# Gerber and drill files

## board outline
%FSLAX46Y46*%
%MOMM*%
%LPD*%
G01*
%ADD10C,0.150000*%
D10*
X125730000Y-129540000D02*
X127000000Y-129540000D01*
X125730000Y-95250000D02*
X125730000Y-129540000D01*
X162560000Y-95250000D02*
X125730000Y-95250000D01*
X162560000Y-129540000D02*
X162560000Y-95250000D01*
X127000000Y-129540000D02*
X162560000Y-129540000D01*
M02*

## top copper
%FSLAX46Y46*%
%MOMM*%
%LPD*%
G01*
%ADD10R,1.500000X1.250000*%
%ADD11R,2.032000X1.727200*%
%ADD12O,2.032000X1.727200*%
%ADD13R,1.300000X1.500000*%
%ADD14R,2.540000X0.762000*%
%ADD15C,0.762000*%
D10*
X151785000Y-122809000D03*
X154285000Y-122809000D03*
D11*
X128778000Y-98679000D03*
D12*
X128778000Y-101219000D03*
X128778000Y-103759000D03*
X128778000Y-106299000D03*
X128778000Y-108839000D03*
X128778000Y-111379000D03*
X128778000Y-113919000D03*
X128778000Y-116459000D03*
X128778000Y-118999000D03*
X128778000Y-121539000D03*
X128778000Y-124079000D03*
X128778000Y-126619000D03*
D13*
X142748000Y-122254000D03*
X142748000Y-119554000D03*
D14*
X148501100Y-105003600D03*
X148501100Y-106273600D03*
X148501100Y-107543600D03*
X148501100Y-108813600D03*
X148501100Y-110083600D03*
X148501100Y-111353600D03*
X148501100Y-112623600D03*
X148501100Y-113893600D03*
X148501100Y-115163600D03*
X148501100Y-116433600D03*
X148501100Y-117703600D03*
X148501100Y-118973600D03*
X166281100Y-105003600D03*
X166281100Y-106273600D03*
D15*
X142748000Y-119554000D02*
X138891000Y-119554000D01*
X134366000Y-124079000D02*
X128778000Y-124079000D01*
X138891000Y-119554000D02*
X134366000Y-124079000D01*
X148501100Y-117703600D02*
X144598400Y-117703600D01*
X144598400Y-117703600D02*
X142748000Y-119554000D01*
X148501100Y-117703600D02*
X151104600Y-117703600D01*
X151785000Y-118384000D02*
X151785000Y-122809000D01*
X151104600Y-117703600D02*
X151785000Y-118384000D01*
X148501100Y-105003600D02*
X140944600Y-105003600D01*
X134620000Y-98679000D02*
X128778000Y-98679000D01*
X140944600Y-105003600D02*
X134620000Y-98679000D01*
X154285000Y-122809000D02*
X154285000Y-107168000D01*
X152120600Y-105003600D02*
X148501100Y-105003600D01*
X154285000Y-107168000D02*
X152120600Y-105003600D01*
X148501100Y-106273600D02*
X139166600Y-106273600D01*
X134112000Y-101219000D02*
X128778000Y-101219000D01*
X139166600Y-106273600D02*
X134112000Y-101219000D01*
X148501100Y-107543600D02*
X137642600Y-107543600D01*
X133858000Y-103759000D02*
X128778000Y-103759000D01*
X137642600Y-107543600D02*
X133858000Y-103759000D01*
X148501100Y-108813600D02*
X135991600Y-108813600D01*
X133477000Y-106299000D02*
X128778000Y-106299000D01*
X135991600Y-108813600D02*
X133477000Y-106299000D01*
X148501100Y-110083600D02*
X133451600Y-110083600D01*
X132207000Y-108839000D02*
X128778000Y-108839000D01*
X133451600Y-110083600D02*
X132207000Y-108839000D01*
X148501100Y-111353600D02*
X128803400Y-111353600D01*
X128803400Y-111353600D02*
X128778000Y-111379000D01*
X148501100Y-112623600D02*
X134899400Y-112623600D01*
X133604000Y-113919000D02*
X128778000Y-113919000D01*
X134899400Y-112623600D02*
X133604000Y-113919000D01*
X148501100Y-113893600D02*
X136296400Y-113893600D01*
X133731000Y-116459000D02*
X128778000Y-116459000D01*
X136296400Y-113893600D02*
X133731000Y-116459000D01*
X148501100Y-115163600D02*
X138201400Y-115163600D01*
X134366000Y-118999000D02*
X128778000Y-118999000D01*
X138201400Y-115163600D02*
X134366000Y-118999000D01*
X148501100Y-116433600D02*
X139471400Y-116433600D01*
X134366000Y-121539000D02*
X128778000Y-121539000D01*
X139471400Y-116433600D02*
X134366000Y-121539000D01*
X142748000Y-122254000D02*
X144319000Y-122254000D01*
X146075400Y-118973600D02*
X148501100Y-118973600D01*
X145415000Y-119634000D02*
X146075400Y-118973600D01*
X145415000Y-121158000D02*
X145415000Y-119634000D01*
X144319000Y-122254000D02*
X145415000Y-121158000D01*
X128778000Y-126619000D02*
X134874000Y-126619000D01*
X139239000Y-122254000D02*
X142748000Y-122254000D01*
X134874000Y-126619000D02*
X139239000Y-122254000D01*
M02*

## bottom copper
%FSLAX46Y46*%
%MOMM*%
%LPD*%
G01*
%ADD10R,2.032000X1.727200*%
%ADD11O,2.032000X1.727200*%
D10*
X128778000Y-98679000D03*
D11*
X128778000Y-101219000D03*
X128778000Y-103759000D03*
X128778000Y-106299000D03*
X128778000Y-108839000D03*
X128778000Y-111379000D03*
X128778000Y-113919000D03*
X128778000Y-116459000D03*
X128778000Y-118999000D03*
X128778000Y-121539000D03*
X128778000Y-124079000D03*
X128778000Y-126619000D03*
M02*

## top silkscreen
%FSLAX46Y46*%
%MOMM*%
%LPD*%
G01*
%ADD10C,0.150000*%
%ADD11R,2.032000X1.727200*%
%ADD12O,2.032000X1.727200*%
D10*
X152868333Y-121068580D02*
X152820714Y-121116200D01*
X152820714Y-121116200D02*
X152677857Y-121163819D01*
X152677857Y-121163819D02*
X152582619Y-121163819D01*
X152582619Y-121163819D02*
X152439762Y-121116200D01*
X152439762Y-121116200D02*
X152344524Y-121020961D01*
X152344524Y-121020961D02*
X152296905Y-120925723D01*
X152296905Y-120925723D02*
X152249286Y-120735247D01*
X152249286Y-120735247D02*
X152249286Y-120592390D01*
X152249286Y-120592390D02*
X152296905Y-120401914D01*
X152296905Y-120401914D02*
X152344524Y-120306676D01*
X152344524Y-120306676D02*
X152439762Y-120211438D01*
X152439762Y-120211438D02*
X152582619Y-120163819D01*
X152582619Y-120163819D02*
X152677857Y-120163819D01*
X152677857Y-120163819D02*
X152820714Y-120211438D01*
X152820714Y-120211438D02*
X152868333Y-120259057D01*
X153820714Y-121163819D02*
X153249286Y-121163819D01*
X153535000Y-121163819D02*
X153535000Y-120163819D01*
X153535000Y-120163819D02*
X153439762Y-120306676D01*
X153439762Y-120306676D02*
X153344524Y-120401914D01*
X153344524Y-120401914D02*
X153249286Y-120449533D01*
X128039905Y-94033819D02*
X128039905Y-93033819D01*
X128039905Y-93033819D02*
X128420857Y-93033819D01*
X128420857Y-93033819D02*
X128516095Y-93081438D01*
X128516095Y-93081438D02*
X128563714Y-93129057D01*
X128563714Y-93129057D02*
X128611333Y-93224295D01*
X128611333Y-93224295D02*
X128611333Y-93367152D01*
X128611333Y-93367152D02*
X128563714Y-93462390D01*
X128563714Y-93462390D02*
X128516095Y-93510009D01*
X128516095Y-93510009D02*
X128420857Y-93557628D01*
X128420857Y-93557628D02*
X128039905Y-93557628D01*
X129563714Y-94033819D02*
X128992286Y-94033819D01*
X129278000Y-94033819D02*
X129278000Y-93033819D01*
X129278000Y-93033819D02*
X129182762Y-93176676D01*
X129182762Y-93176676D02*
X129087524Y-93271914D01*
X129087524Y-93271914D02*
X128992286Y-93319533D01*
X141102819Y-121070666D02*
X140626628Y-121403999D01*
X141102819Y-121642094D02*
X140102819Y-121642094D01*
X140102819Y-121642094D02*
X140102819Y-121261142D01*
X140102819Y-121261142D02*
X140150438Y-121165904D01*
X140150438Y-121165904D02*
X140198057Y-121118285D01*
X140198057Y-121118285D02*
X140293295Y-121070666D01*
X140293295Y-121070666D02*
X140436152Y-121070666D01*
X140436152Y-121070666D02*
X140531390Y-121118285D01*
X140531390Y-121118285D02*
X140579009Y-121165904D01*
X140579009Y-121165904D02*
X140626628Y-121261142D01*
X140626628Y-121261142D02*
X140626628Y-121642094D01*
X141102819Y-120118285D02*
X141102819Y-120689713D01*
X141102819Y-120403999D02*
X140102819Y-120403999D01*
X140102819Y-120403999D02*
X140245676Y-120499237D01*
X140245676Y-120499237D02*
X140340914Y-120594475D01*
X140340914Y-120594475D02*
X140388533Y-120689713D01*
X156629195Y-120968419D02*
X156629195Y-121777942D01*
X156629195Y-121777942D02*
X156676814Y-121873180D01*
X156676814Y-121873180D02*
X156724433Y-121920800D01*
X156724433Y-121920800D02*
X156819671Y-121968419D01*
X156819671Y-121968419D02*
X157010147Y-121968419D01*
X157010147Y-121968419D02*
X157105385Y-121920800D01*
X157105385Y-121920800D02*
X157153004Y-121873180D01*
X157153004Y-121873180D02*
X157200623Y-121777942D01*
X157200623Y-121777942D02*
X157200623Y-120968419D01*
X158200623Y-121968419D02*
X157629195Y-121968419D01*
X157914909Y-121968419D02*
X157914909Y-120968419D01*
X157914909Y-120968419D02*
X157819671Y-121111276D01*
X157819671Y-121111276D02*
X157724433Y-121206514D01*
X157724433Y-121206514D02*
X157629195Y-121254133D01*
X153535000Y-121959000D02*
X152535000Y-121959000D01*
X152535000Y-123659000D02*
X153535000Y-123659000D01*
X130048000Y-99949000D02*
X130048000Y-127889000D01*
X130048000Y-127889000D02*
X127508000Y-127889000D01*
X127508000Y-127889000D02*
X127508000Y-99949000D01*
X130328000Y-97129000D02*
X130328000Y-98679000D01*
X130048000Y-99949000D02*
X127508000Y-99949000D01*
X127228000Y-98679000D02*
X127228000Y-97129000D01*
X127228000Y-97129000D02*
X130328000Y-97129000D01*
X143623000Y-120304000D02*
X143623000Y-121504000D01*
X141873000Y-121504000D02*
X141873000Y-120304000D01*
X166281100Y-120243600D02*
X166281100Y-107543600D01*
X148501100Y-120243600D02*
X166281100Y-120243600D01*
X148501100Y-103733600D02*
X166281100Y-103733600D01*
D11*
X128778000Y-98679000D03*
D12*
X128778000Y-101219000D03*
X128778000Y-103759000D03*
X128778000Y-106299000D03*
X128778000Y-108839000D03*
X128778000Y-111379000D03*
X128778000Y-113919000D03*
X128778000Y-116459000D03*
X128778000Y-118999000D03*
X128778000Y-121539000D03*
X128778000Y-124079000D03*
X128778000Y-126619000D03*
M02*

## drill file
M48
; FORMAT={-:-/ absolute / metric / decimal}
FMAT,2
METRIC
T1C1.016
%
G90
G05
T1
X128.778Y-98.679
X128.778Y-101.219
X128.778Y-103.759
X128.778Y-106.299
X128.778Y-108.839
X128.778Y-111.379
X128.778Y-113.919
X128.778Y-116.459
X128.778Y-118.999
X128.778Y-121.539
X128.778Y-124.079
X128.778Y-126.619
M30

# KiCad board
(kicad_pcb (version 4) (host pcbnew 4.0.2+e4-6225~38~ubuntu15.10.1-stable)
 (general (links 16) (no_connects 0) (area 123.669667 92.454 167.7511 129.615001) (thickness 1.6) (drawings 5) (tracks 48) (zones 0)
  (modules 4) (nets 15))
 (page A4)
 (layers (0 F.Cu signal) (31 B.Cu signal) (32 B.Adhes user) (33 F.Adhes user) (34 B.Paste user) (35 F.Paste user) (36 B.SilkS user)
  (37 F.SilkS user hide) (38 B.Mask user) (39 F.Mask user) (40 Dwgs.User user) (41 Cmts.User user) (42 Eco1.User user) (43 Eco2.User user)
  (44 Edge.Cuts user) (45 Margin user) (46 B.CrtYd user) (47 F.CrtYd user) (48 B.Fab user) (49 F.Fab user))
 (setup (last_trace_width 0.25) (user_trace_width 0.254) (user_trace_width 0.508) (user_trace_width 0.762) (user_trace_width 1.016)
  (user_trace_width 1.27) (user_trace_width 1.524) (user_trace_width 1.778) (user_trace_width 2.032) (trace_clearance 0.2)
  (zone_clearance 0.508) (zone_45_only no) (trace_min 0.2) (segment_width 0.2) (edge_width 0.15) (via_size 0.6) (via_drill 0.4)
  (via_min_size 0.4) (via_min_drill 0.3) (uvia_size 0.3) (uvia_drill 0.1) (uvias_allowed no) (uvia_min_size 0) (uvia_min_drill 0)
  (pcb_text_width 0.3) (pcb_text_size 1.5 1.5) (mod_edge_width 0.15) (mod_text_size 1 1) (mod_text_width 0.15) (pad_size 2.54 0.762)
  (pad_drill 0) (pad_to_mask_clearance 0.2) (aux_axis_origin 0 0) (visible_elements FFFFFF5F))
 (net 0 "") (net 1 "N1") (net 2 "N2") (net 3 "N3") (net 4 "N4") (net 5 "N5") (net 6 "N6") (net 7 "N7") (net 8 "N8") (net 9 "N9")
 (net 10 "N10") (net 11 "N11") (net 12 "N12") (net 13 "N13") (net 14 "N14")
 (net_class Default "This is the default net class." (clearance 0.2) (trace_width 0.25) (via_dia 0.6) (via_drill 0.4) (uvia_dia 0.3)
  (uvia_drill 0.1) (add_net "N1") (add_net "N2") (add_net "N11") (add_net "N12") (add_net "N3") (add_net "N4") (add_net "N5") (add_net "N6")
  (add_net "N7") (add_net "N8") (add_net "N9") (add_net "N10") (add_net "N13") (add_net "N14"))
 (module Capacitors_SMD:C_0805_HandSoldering (layer F.Cu) (at 153.035 122.809)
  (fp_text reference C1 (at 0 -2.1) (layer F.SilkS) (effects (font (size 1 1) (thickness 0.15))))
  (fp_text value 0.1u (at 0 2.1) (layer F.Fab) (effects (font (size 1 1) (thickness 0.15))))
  (fp_line (start 0.5 -0.85) (end -0.5 -0.85) (layer F.SilkS) (width 0.15))
  (fp_line (start -0.5 0.85) (end 0.5 0.85) (layer F.SilkS) (width 0.15))
  (pad 1 smd rect (at -1.25 0) (size 1.5 1.25) (layers F.Cu F.Paste F.Mask) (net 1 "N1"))
  (pad 2 smd rect (at 1.25 0) (size 1.5 1.25) (layers F.Cu F.Paste F.Mask) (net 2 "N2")))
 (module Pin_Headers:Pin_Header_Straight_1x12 (layer F.Cu) (at 128.778 98.679)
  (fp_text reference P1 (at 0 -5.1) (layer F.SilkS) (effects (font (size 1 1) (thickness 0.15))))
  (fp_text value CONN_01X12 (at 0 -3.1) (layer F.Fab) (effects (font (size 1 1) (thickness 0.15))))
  (fp_line (start 1.27 1.27) (end 1.27 29.21) (layer F.SilkS) (width 0.15))
  (fp_line (start 1.27 29.21) (end -1.27 29.21) (layer F.SilkS) (width 0.15))
  (fp_line (start -1.27 29.21) (end -1.27 1.27) (layer F.SilkS) (width 0.15))
  (fp_line (start 1.55 -1.55) (end 1.55 0) (layer F.SilkS) (width 0.15))
  (fp_line (start 1.27 1.27) (end -1.27 1.27) (layer F.SilkS) (width 0.15))
  (fp_line (start -1.55 0) (end -1.55 -1.55) (layer F.SilkS) (width 0.15))
  (fp_line (start -1.55 -1.55) (end 1.55 -1.55) (layer F.SilkS) (width 0.15))
  (pad 1 thru_hole rect (at 0 0) (size 2.032 1.7272) (drill 1.016) (layers *.Cu *.Mask F.SilkS) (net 2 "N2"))
  (pad 2 thru_hole oval (at 0 2.54) (size 2.032 1.7272) (drill 1.016) (layers *.Cu *.Mask F.SilkS) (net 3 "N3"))
  (pad 3 thru_hole oval (at 0 5.08) (size 2.032 1.7272) (drill 1.016) (layers *.Cu *.Mask F.SilkS) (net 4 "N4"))
  (pad 4 thru_hole oval (at 0 7.62) (size 2.032 1.7272) (drill 1.016) (layers *.Cu *.Mask F.SilkS) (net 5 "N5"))
  (pad 5 thru_hole oval (at 0 10.16) (size 2.032 1.7272) (drill 1.016) (layers *.Cu *.Mask F.SilkS) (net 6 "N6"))
  (pad 6 thru_hole oval (at 0 12.7) (size 2.032 1.7272) (drill 1.016) (layers *.Cu *.Mask F.SilkS) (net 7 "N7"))
  (pad 7 thru_hole oval (at 0 15.24) (size 2.032 1.7272) (drill 1.016) (layers *.Cu *.Mask F.SilkS) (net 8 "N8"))
  (pad 8 thru_hole oval (at 0 17.78) (size 2.032 1.7272) (drill 1.016) (layers *.Cu *.Mask F.SilkS) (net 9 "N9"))
  (pad 9 thru_hole oval (at 0 20.32) (size 2.032 1.7272) (drill 1.016) (layers *.Cu *.Mask F.SilkS) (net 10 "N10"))
  (pad 10 thru_hole oval (at 0 22.86) (size 2.032 1.7272) (drill 1.016) (layers *.Cu *.Mask F.SilkS) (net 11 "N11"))
  (pad 11 thru_hole oval (at 0 25.4) (size 2.032 1.7272) (drill 1.016) (layers *.Cu *.Mask F.SilkS) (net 1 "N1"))
  (pad 12 thru_hole oval (at 0 27.94) (size 2.032 1.7272) (drill 1.016) (layers *.Cu *.Mask F.SilkS) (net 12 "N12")))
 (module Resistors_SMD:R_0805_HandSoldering (layer F.Cu) (at 142.748 120.904 90)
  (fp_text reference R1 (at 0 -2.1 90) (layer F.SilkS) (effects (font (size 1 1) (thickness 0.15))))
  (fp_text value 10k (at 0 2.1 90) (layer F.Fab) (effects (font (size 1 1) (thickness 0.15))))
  (fp_line (start 0.6 0.875) (end -0.6 0.875) (layer F.SilkS) (width 0.15))
  (fp_line (start -0.6 -0.875) (end 0.6 -0.875) (layer F.SilkS) (width 0.15))
  (pad 1 smd rect (at -1.35 0 90) (size 1.5 1.3) (layers F.Cu F.Paste F.Mask) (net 12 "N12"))
  (pad 2 smd rect (at 1.35 0 90) (size 1.5 1.3) (layers F.Cu F.Paste F.Mask) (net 1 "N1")))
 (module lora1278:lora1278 (layer F.Cu) (at 148.5011 105.0036)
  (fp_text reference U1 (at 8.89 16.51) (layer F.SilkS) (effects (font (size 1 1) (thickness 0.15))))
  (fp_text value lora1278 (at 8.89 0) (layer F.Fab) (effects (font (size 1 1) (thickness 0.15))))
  (fp_line (start 17.78 15.24) (end 17.78 2.54) (layer F.SilkS) (width 0.15))
  (fp_line (start 0 15.24) (end 17.78 15.24) (layer F.SilkS) (width 0.15))
  (fp_line (start 0 -1.27) (end 17.78 -1.27) (layer F.SilkS) (width 0.15))
  (pad 1 smd rect (at 0 0) (size 2.54 0.762) (layers F.Cu F.Paste F.Mask) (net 2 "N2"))
  (pad 2 smd rect (at 0 1.27) (size 2.54 0.762) (layers F.Cu F.Paste F.Mask) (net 3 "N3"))
  (pad 3 smd rect (at 0 2.54) (size 2.54 0.762) (layers F.Cu F.Paste F.Mask) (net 4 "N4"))
  (pad 4 smd rect (at 0 3.81) (size 2.54 0.762) (layers F.Cu F.Paste F.Mask) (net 5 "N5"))
  (pad 5 smd rect (at 0 5.08) (size 2.54 0.762) (layers F.Cu F.Paste F.Mask) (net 6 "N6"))
  (pad 6 smd rect (at 0 6.35) (size 2.54 0.762) (layers F.Cu F.Paste F.Mask) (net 7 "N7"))
  (pad 7 smd rect (at 0 7.62) (size 2.54 0.762) (layers F.Cu F.Paste F.Mask) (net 8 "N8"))
  (pad 8 smd rect (at 0 8.89) (size 2.54 0.762) (layers F.Cu F.Paste F.Mask) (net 9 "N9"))
  (pad 9 smd rect (at 0 10.16) (size 2.54 0.762) (layers F.Cu F.Paste F.Mask) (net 10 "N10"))
  (pad 10 smd rect (at 0 11.43) (size 2.54 0.762) (layers F.Cu F.Paste F.Mask) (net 11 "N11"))
  (pad 11 smd rect (at 0 12.7) (size 2.54 0.762) (layers F.Cu F.Paste F.Mask) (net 1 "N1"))
  (pad 12 smd rect (at 0 13.97) (size 2.54 0.762) (layers F.Cu F.Paste F.Mask) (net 12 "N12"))
  (pad 13 smd rect (at 17.78 0) (size 2.54 0.762) (layers F.Cu F.Paste F.Mask) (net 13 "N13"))
  (pad 14 smd rect (at 17.78 1.27) (size 2.54 0.762) (layers F.Cu F.Paste F.Mask) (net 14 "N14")))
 (gr_line (start 125.73 129.54) (end 127 129.54) (angle 90) (layer Edge.Cuts) (width 0.15))
 (gr_line (start 125.73 95.25) (end 125.73 129.54) (angle 90) (layer Edge.Cuts) (width 0.15))
 (gr_line (start 162.56 95.25) (end 125.73 95.25) (angle 90) (layer Edge.Cuts) (width 0.15))
 (gr_line (start 162.56 129.54) (end 162.56 95.25) (angle 90) (layer Edge.Cuts) (width 0.15))
 (gr_line (start 127 129.54) (end 162.56 129.54) (angle 90) (layer Edge.Cuts) (width 0.15))
 (segment (start 142.748 119.554) (end 138.891 119.554) (width 0.762) (layer F.Cu) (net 1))
 (segment (start 134.366 124.079) (end 128.778 124.079) (width 0.762) (layer F.Cu) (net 1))
 (segment (start 138.891 119.554) (end 134.366 124.079) (width 0.762) (layer F.Cu) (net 1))
 (segment (start 148.5011 117.7036) (end 144.5984 117.7036) (width 0.762) (layer F.Cu) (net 1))
 (segment (start 144.5984 117.7036) (end 142.748 119.554) (width 0.762) (layer F.Cu) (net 1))
 (segment (start 148.5011 117.7036) (end 151.1046 117.7036) (width 0.762) (layer F.Cu) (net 1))
 (segment (start 151.785 118.384) (end 151.785 122.809) (width 0.762) (layer F.Cu) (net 1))
 (segment (start 151.1046 117.7036) (end 151.785 118.384) (width 0.762) (layer F.Cu) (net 1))
 (segment (start 148.5011 105.0036) (end 140.9446 105.0036) (width 0.762) (layer F.Cu) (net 2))
 (segment (start 134.62 98.679) (end 128.778 98.679) (width 0.762) (layer F.Cu) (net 2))
 (segment (start 140.9446 105.0036) (end 134.62 98.679) (width 0.762) (layer F.Cu) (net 2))
 (segment (start 154.285 122.809) (end 154.285 107.168) (width 0.762) (layer F.Cu) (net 2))
 (segment (start 152.1206 105.0036) (end 148.5011 105.0036) (width 0.762) (layer F.Cu) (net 2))
 (segment (start 154.285 107.168) (end 152.1206 105.0036) (width 0.762) (layer F.Cu) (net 2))
 (segment (start 148.5011 106.2736) (end 139.1666 106.2736) (width 0.762) (layer F.Cu) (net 3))
 (segment (start 134.112 101.219) (end 128.778 101.219) (width 0.762) (layer F.Cu) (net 3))
 (segment (start 139.1666 106.2736) (end 134.112 101.219) (width 0.762) (layer F.Cu) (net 3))
 (segment (start 148.5011 107.5436) (end 137.6426 107.5436) (width 0.762) (layer F.Cu) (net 4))
 (segment (start 133.858 103.759) (end 128.778 103.759) (width 0.762) (layer F.Cu) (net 4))
 (segment (start 137.6426 107.5436) (end 133.858 103.759) (width 0.762) (layer F.Cu) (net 4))
 (segment (start 148.5011 108.8136) (end 135.9916 108.8136) (width 0.762) (layer F.Cu) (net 5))
 (segment (start 133.477 106.299) (end 128.778 106.299) (width 0.762) (layer F.Cu) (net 5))
 (segment (start 135.9916 108.8136) (end 133.477 106.299) (width 0.762) (layer F.Cu) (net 5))
 (segment (start 148.5011 110.0836) (end 133.4516 110.0836) (width 0.762) (layer F.Cu) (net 6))
 (segment (start 132.207 108.839) (end 128.778 108.839) (width 0.762) (layer F.Cu) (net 6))
 (segment (start 133.4516 110.0836) (end 132.207 108.839) (width 0.762) (layer F.Cu) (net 6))
 (segment (start 148.5011 111.3536) (end 128.8034 111.3536) (width 0.762) (layer F.Cu) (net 7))
 (segment (start 128.8034 111.3536) (end 128.778 111.379) (width 0.762) (layer F.Cu) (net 7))
 (segment (start 148.5011 112.6236) (end 134.8994 112.6236) (width 0.762) (layer F.Cu) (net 8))
 (segment (start 133.604 113.919) (end 128.778 113.919) (width 0.762) (layer F.Cu) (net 8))
 (segment (start 134.8994 112.6236) (end 133.604 113.919) (width 0.762) (layer F.Cu) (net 8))
 (segment (start 148.5011 113.8936) (end 136.2964 113.8936) (width 0.762) (layer F.Cu) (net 9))
 (segment (start 133.731 116.459) (end 128.778 116.459) (width 0.762) (layer F.Cu) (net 9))
 (segment (start 136.2964 113.8936) (end 133.731 116.459) (width 0.762) (layer F.Cu) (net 9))
 (segment (start 148.5011 115.1636) (end 138.2014 115.1636) (width 0.762) (layer F.Cu) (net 10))
 (segment (start 134.366 118.999) (end 128.778 118.999) (width 0.762) (layer F.Cu) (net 10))
 (segment (start 138.2014 115.1636) (end 134.366 118.999) (width 0.762) (layer F.Cu) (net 10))
 (segment (start 148.5011 116.4336) (end 139.4714 116.4336) (width 0.762) (layer F.Cu) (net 11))
 (segment (start 134.366 121.539) (end 128.778 121.539) (width 0.762) (layer F.Cu) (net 11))
 (segment (start 139.4714 116.4336) (end 134.366 121.539) (width 0.762) (layer F.Cu) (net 11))
 (segment (start 142.748 122.254) (end 144.319 122.254) (width 0.762) (layer F.Cu) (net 12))
 (segment (start 146.0754 118.9736) (end 148.5011 118.9736) (width 0.762) (layer F.Cu) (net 12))
 (segment (start 145.415 119.634) (end 146.0754 118.9736) (width 0.762) (layer F.Cu) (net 12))
 (segment (start 145.415 121.158) (end 145.415 119.634) (width 0.762) (layer F.Cu) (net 12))
 (segment (start 144.319 122.254) (end 145.415 121.158) (width 0.762) (layer F.Cu) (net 12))
 (segment (start 128.778 126.619) (end 134.874 126.619) (width 0.762) (layer F.Cu) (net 12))
 (segment (start 139.239 122.254) (end 142.748 122.254) (width 0.762) (layer F.Cu) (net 12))
 (segment (start 134.874 126.619) (end 139.239 122.254) (width 0.762) (layer F.Cu) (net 12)))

